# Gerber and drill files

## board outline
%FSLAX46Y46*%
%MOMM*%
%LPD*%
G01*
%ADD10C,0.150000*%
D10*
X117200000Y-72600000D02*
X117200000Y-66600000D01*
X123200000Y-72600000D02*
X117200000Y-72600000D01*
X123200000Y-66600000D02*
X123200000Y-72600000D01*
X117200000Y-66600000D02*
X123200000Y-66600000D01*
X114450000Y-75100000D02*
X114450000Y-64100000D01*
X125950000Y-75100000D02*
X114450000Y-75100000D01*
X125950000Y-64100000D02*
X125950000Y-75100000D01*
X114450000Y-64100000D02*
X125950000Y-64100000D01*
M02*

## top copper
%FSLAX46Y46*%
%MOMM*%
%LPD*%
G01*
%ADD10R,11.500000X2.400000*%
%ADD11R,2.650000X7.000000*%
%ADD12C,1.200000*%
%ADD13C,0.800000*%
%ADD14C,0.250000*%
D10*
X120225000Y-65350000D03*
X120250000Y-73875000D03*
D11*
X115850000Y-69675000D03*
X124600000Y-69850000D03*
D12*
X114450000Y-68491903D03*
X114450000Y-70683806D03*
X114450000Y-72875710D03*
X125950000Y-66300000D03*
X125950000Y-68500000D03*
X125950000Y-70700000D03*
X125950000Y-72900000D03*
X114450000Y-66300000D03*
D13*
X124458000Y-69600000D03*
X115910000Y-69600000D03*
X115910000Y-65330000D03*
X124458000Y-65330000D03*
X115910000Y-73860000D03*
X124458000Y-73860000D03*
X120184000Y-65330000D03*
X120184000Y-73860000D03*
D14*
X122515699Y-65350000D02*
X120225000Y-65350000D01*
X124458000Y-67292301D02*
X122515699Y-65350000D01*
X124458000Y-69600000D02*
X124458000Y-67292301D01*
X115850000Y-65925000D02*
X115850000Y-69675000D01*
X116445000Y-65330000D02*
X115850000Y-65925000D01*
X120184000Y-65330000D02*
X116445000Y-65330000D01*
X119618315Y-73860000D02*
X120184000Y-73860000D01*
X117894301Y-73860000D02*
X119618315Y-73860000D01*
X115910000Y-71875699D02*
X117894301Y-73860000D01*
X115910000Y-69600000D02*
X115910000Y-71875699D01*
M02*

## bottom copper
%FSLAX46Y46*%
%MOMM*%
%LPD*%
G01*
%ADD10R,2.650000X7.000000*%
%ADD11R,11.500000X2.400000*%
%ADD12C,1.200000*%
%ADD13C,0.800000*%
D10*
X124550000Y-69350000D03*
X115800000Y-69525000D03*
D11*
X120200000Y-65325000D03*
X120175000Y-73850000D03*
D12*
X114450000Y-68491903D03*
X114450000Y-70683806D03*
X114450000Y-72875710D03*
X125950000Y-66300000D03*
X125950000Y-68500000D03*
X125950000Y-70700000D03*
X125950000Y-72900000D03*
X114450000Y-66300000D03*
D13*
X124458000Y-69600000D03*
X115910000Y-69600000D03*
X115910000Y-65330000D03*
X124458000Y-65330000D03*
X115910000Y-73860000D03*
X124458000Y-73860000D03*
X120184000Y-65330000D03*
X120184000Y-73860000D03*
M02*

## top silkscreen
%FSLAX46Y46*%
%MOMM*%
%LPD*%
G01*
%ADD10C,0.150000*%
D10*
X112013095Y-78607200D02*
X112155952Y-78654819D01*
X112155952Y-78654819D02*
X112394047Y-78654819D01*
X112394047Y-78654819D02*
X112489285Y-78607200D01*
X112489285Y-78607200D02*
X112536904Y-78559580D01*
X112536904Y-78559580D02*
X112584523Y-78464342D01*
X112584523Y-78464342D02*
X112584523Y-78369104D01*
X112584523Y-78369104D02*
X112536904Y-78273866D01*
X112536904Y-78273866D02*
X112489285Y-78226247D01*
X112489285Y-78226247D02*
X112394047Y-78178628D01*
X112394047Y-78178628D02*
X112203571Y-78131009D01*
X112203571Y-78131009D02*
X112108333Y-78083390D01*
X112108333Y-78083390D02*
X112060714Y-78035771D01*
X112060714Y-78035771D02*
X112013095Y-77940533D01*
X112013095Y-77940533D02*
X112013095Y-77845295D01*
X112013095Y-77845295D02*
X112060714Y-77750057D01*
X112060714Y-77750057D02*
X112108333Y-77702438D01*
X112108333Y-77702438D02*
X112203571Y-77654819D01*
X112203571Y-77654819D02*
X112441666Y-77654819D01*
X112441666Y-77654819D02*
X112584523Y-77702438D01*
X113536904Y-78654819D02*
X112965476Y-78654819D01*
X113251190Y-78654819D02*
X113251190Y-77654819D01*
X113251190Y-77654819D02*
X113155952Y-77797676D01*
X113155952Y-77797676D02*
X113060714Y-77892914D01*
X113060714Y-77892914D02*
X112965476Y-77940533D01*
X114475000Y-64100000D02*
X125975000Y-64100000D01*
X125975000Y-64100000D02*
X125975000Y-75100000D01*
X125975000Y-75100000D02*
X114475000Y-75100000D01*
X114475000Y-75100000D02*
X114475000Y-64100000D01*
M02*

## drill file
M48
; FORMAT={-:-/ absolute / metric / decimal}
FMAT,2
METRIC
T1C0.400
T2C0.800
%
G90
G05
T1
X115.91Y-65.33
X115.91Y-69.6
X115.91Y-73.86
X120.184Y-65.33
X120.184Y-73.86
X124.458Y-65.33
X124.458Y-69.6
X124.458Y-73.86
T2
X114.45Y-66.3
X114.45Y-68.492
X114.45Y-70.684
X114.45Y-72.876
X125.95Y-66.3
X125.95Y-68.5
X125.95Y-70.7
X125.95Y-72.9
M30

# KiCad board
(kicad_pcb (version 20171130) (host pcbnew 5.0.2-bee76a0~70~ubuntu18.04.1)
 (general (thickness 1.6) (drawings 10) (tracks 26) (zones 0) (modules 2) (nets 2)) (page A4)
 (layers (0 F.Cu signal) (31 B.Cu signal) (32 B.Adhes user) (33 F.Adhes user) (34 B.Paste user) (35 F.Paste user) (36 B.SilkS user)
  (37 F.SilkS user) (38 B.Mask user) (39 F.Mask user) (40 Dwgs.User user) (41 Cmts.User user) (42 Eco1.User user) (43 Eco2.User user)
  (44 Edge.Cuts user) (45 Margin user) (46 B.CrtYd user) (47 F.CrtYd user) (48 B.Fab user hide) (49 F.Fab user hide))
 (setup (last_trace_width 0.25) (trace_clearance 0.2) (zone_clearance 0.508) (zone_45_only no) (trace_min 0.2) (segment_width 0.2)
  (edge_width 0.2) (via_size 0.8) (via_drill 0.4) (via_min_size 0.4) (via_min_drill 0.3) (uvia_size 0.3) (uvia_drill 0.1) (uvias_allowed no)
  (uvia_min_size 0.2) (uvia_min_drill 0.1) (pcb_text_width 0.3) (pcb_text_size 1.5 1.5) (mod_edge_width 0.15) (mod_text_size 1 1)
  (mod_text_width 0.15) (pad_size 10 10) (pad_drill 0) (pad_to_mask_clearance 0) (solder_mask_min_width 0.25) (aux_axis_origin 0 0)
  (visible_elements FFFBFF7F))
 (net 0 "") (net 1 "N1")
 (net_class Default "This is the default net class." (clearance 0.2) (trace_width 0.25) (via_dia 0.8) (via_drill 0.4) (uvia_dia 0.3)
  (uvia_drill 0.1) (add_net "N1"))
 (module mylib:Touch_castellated (layer F.Cu) (at 114.475 64.1)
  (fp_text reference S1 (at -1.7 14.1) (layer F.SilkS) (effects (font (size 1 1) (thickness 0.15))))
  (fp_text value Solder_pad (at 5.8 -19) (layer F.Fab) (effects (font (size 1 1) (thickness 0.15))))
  (fp_line (start 0 0) (end 11.5 0) (layer F.SilkS) (width 0.15))
  (fp_line (start 11.5 0) (end 11.5 11) (layer F.SilkS) (width 0.15))
  (fp_line (start 11.5 11) (end 0 11) (layer F.SilkS) (width 0.15))
  (fp_line (start 0 11) (end 0 0) (layer F.SilkS) (width 0.15))
  (pad 1 smd rect (at 5.75 1.25) (size 11.5 2.4) (layers F.Cu F.Paste F.Mask) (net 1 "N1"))
  (pad 1 smd rect (at 5.775 9.775) (size 11.5 2.4) (layers F.Cu F.Paste F.Mask) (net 1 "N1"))
  (pad 1 smd rect (at 1.375 5.575) (size 2.65 7) (layers F.Cu F.Paste F.Mask) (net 1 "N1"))
  (pad 1 smd rect (at 10.125 5.75) (size 2.65 7) (layers F.Cu F.Paste F.Mask) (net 1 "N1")))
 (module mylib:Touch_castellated (layer B.Cu) (at 114.425 75.1)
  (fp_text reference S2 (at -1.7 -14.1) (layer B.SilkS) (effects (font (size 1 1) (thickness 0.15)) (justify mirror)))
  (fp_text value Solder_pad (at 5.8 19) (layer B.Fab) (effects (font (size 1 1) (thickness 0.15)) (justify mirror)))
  (pad 1 smd rect (at 10.125 -5.75) (size 2.65 7) (layers B.Cu B.Paste B.Mask) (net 1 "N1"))
  (pad 1 smd rect (at 1.375 -5.575) (size 2.65 7) (layers B.Cu B.Paste B.Mask) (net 1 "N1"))
  (pad 1 smd rect (at 5.775 -9.775) (size 11.5 2.4) (layers B.Cu B.Paste B.Mask) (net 1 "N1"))
  (pad 1 smd rect (at 5.75 -1.25) (size 11.5 2.4) (layers B.Cu B.Paste B.Mask) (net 1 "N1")))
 (gr_line (start 117.2 72.6) (end 117.2 66.6) (layer Edge.Cuts) (width 0.15))
 (gr_line (start 123.2 72.6) (end 117.2 72.6) (layer Edge.Cuts) (width 0.15))
 (gr_line (start 123.2 66.6) (end 123.2 72.6) (layer Edge.Cuts) (width 0.15))
 (gr_line (start 117.2 66.6) (end 123.2 66.6) (layer Edge.Cuts) (width 0.15))
 (gr_line (start 114.45 75.1) (end 114.45 64.1) (layer Edge.Cuts) (width 0.15))
 (gr_line (start 125.95 75.1) (end 114.45 75.1) (layer Edge.Cuts) (width 0.15))
 (gr_line (start 125.95 64.1) (end 125.95 75.1) (layer Edge.Cuts) (width 0.15))
 (gr_line (start 114.45 64.1) (end 125.95 64.1) (layer Edge.Cuts) (width 0.15))
 (via (at 114.45 68.491903) (size 1.2) (drill 0.8) (layers F.Cu B.Cu) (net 1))
 (via (at 114.45 70.683806) (size 1.2) (drill 0.8) (layers F.Cu B.Cu) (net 1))
 (via (at 114.45 72.87571) (size 1.2) (drill 0.8) (layers F.Cu B.Cu) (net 1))
 (via (at 125.95 66.3) (size 1.2) (drill 0.8) (layers F.Cu B.Cu) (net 1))
 (via (at 125.95 68.5) (size 1.2) (drill 0.8) (layers F.Cu B.Cu) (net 1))
 (via (at 125.95 70.7) (size 1.2) (drill 0.8) (layers F.Cu B.Cu) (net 1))
 (via (at 125.95 72.9) (size 1.2) (drill 0.8) (layers F.Cu B.Cu) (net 1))
 (via (at 114.45 66.3) (size 1.2) (drill 0.8) (layers F.Cu B.Cu) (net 1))
 (via (at 124.458 69.6) (size 0.8) (drill 0.4) (layers F.Cu B.Cu) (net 1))
 (via (at 115.91 69.6) (size 0.8) (drill 0.4) (layers F.Cu B.Cu) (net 1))
 (via (at 115.91 65.33) (size 0.8) (drill 0.4) (layers F.Cu B.Cu) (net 1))
 (via (at 124.458 65.33) (size 0.8) (drill 0.4) (layers F.Cu B.Cu) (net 1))
 (via (at 115.91 73.86) (size 0.8) (drill 0.4) (layers F.Cu B.Cu) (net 1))
 (via (at 124.458 73.86) (size 0.8) (drill 0.4) (layers F.Cu B.Cu) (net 1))
 (via (at 120.184 65.33) (size 0.8) (drill 0.4) (layers F.Cu B.Cu) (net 1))
 (via (at 120.184 73.86) (size 0.8) (drill 0.4) (layers F.Cu B.Cu) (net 1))
 (segment (start 122.515699 65.35) (end 120.225 65.35) (width 0.25) (layer F.Cu) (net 1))
 (segment (start 124.458 67.292301) (end 122.515699 65.35) (width 0.25) (layer F.Cu) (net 1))
 (segment (start 124.458 69.6) (end 124.458 67.292301) (width 0.25) (layer F.Cu) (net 1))
 (segment (start 115.85 65.925) (end 115.85 69.675) (width 0.25) (layer F.Cu) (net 1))
 (segment (start 116.445 65.33) (end 115.85 65.925) (width 0.25) (layer F.Cu) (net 1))
 (segment (start 120.184 65.33) (end 116.445 65.33) (width 0.25) (layer F.Cu) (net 1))
 (segment (start 119.618315 73.86) (end 120.184 73.86) (width 0.25) (layer F.Cu) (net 1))
 (segment (start 117.894301 73.86) (end 119.618315 73.86) (width 0.25) (layer F.Cu) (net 1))
 (segment (start 115.91 71.875699) (end 117.894301 73.86) (width 0.25) (layer F.Cu) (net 1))
 (segment (start 115.91 69.6) (end 115.91 71.875699) (width 0.25) (layer F.Cu) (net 1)))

